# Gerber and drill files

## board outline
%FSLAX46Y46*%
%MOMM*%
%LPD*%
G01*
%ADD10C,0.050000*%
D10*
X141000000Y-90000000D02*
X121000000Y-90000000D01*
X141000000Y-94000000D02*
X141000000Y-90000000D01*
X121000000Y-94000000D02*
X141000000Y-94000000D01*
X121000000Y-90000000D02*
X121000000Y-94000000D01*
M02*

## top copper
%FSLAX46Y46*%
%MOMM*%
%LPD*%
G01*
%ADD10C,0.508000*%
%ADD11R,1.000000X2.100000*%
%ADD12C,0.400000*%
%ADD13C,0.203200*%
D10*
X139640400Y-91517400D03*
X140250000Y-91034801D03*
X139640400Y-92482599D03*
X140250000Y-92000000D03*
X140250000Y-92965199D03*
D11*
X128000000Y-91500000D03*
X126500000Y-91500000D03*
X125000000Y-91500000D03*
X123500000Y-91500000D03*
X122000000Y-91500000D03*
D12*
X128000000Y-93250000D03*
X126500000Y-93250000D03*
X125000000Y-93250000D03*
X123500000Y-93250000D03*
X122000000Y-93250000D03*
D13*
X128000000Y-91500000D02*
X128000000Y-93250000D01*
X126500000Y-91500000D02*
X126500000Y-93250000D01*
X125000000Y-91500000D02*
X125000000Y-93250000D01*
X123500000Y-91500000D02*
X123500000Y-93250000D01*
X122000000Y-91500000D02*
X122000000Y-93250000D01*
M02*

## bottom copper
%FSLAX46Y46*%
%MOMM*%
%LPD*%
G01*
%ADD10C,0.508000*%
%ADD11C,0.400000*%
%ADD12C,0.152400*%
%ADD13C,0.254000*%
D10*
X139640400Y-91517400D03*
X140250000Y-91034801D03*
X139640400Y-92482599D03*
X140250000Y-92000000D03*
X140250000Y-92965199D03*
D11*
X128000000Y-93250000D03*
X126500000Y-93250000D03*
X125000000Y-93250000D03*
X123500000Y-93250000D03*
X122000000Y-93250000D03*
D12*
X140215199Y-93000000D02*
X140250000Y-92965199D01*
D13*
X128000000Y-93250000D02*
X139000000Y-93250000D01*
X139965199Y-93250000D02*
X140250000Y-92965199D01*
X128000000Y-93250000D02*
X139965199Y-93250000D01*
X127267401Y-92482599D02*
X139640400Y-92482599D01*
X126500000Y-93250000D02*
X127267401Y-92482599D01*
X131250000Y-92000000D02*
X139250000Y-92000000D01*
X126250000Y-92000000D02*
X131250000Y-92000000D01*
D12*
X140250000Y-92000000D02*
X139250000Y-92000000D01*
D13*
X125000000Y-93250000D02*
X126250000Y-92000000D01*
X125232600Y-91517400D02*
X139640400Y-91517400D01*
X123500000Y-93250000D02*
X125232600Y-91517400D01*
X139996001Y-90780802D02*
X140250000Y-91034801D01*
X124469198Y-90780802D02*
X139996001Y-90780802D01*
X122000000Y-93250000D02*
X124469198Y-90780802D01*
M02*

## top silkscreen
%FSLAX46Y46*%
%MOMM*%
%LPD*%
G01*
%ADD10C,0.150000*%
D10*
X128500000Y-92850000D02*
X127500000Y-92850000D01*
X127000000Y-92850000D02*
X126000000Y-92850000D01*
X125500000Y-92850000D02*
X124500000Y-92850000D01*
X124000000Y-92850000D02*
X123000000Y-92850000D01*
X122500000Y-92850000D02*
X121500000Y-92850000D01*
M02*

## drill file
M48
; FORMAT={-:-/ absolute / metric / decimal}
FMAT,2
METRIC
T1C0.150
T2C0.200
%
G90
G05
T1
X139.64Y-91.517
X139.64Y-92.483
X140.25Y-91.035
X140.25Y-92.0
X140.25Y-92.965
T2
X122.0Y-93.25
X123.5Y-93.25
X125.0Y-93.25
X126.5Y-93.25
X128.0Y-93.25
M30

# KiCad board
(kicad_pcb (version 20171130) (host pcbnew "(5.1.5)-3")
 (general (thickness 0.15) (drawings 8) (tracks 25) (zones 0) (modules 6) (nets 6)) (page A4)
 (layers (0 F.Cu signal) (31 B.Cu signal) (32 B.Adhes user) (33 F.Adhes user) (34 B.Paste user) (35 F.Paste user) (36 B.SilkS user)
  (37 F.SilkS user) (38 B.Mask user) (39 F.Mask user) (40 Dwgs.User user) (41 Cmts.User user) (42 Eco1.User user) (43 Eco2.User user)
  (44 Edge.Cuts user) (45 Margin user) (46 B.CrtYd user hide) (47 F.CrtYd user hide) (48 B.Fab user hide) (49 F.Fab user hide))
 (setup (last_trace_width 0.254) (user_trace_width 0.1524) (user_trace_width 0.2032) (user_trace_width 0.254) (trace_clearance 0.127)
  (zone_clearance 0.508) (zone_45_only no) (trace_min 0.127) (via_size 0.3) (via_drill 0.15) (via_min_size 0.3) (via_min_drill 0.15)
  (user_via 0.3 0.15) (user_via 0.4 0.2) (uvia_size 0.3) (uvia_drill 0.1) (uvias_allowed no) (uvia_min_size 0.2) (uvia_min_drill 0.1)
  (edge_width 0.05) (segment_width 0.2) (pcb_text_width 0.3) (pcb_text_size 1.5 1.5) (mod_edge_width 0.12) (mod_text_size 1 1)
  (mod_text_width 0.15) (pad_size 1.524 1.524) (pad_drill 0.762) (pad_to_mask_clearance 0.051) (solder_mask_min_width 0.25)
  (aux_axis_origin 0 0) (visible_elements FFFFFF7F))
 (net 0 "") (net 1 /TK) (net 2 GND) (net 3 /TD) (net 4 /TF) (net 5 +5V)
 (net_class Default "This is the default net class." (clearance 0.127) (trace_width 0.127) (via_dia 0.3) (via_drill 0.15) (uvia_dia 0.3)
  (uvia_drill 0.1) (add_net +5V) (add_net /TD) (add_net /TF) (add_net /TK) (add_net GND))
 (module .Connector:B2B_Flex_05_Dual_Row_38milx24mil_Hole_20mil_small (layer F.Cu) (at 140.225 91.009801 270)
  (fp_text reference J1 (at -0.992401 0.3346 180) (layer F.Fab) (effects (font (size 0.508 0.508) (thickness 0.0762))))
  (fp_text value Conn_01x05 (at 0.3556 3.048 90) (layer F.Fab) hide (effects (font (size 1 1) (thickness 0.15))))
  (pad 2 thru_hole circle (at 0.507599 0.5846 270) (size 0.508 0.508) (drill 0.15) (layers *.Cu *.Mask) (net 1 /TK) (zone_connect 2))
  (pad 1 thru_hole circle (at 0.025 -0.025 270) (size 0.508 0.508) (drill 0.15) (layers *.Cu *.Mask) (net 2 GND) (zone_connect 2))
  (pad 4 thru_hole circle (at 1.472798 0.5846 270) (size 0.508 0.508) (drill 0.15) (layers *.Cu *.Mask) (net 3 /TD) (zone_connect 2))
  (pad 3 thru_hole circle (at 0.990199 -0.025 270) (size 0.508 0.508) (drill 0.15) (layers *.Cu *.Mask) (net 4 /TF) (zone_connect 2))
  (pad 5 thru_hole circle (at 1.955398 -0.025 270) (size 0.508 0.508) (drill 0.15) (layers *.Cu *.Mask) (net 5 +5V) (zone_connect 2)))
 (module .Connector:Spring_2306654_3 (layer F.Cu) (at 128 91.5 270)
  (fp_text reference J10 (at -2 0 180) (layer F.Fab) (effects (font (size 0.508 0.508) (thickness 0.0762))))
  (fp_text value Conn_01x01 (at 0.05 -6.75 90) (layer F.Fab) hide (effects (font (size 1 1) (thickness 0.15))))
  (fp_line (start 1.35 -0.5) (end 1.35 0.5) (layer F.SilkS) (width 0.15))
  (pad 1 smd rect (at 0 0 270) (size 2.1 1) (layers F.Cu F.Paste F.Mask) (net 5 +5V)))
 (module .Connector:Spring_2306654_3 (layer F.Cu) (at 126.5 91.5 270)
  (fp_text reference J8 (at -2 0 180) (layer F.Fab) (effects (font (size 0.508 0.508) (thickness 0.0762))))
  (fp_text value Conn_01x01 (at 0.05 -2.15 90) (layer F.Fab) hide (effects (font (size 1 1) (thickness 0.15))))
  (fp_line (start 1.35 -0.5) (end 1.35 0.5) (layer F.SilkS) (width 0.15))
  (pad 1 smd rect (at 0 0 270) (size 2.1 1) (layers F.Cu F.Paste F.Mask) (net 3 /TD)))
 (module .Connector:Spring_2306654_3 (layer F.Cu) (at 125 91.5 270)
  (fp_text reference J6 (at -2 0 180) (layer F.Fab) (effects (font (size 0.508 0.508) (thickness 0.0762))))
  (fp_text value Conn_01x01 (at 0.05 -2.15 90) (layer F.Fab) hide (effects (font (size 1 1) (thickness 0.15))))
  (fp_line (start 1.35 -0.5) (end 1.35 0.5) (layer F.SilkS) (width 0.15))
  (pad 1 smd rect (at 0 0 270) (size 2.1 1) (layers F.Cu F.Paste F.Mask) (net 4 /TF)))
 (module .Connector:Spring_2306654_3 (layer F.Cu) (at 123.5 91.5 270)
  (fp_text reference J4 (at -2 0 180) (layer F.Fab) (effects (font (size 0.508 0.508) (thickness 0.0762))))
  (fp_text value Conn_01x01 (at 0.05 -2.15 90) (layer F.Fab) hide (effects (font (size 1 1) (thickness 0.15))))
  (fp_line (start 1.35 -0.5) (end 1.35 0.5) (layer F.SilkS) (width 0.15))
  (pad 1 smd rect (at 0 0 270) (size 2.1 1) (layers F.Cu F.Paste F.Mask) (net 1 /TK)))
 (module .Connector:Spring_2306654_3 (layer F.Cu) (at 122 91.5 270)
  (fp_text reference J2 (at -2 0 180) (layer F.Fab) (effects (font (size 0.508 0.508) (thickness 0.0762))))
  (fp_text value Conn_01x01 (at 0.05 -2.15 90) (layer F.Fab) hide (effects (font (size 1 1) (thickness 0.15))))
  (fp_line (start 1.35 -0.5) (end 1.35 0.5) (layer F.SilkS) (width 0.15))
  (pad 1 smd rect (at 0 0 270) (size 2.1 1) (layers F.Cu F.Paste F.Mask) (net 2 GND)))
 (gr_line (start 141 90) (end 121 90) (layer Edge.Cuts) (width 0.05))
 (gr_line (start 141 94) (end 141 90) (layer Edge.Cuts) (width 0.05))
 (gr_line (start 121 94) (end 141 94) (layer Edge.Cuts) (width 0.05))
 (gr_line (start 121 90) (end 121 94) (layer Edge.Cuts) (width 0.05))
 (segment (start 140.215199 93) (end 140.25 92.965199) (width 0.1524) (layer B.Cu) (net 5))
 (segment (start 128 93.25) (end 139 93.25) (width 0.254) (layer B.Cu) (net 5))
 (segment (start 128 91.5) (end 128 93.25) (width 0.2032) (layer F.Cu) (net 5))
 (via (at 128 93.25) (size 0.4) (drill 0.2) (layers F.Cu B.Cu) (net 5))
 (segment (start 139.965199 93.25) (end 140.25 92.965199) (width 0.254) (layer B.Cu) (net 5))
 (segment (start 128 93.25) (end 139.965199 93.25) (width 0.254) (layer B.Cu) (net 5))
 (segment (start 126.5 91.5) (end 126.5 93.25) (width 0.2032) (layer F.Cu) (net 3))
 (via (at 126.5 93.25) (size 0.4) (drill 0.2) (layers F.Cu B.Cu) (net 3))
 (segment (start 127.267401 92.482599) (end 139.6404 92.482599) (width 0.254) (layer B.Cu) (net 3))
 (segment (start 126.5 93.25) (end 127.267401 92.482599) (width 0.254) (layer B.Cu) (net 3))
 (via (at 125 93.25) (size 0.4) (drill 0.2) (layers F.Cu B.Cu) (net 4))
 (segment (start 125 91.5) (end 125 93.25) (width 0.2032) (layer F.Cu) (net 4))
 (segment (start 131.25 92) (end 139.25 92) (width 0.254) (layer B.Cu) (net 4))
 (segment (start 126.25 92) (end 131.25 92) (width 0.254) (layer B.Cu) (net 4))
 (segment (start 140.25 92) (end 139.25 92) (width 0.1524) (layer B.Cu) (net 4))
 (segment (start 125 93.25) (end 126.25 92) (width 0.254) (layer B.Cu) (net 4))
 (via (at 123.5 93.25) (size 0.4) (drill 0.2) (layers F.Cu B.Cu) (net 1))
 (segment (start 123.5 91.5) (end 123.5 93.25) (width 0.2032) (layer F.Cu) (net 1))
 (segment (start 125.2326 91.5174) (end 139.6404 91.5174) (width 0.254) (layer B.Cu) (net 1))
 (segment (start 123.5 93.25) (end 125.2326 91.5174) (width 0.254) (layer B.Cu) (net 1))
 (via (at 122 93.25) (size 0.4) (drill 0.2) (layers F.Cu B.Cu) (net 2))
 (segment (start 122 91.5) (end 122 93.25) (width 0.2032) (layer F.Cu) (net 2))
 (segment (start 139.996001 90.780802) (end 140.25 91.034801) (width 0.254) (layer B.Cu) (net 2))
 (segment (start 124.469198 90.780802) (end 139.996001 90.780802) (width 0.254) (layer B.Cu) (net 2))
 (segment (start 122 93.25) (end 124.469198 90.780802) (width 0.254) (layer B.Cu) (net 2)))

